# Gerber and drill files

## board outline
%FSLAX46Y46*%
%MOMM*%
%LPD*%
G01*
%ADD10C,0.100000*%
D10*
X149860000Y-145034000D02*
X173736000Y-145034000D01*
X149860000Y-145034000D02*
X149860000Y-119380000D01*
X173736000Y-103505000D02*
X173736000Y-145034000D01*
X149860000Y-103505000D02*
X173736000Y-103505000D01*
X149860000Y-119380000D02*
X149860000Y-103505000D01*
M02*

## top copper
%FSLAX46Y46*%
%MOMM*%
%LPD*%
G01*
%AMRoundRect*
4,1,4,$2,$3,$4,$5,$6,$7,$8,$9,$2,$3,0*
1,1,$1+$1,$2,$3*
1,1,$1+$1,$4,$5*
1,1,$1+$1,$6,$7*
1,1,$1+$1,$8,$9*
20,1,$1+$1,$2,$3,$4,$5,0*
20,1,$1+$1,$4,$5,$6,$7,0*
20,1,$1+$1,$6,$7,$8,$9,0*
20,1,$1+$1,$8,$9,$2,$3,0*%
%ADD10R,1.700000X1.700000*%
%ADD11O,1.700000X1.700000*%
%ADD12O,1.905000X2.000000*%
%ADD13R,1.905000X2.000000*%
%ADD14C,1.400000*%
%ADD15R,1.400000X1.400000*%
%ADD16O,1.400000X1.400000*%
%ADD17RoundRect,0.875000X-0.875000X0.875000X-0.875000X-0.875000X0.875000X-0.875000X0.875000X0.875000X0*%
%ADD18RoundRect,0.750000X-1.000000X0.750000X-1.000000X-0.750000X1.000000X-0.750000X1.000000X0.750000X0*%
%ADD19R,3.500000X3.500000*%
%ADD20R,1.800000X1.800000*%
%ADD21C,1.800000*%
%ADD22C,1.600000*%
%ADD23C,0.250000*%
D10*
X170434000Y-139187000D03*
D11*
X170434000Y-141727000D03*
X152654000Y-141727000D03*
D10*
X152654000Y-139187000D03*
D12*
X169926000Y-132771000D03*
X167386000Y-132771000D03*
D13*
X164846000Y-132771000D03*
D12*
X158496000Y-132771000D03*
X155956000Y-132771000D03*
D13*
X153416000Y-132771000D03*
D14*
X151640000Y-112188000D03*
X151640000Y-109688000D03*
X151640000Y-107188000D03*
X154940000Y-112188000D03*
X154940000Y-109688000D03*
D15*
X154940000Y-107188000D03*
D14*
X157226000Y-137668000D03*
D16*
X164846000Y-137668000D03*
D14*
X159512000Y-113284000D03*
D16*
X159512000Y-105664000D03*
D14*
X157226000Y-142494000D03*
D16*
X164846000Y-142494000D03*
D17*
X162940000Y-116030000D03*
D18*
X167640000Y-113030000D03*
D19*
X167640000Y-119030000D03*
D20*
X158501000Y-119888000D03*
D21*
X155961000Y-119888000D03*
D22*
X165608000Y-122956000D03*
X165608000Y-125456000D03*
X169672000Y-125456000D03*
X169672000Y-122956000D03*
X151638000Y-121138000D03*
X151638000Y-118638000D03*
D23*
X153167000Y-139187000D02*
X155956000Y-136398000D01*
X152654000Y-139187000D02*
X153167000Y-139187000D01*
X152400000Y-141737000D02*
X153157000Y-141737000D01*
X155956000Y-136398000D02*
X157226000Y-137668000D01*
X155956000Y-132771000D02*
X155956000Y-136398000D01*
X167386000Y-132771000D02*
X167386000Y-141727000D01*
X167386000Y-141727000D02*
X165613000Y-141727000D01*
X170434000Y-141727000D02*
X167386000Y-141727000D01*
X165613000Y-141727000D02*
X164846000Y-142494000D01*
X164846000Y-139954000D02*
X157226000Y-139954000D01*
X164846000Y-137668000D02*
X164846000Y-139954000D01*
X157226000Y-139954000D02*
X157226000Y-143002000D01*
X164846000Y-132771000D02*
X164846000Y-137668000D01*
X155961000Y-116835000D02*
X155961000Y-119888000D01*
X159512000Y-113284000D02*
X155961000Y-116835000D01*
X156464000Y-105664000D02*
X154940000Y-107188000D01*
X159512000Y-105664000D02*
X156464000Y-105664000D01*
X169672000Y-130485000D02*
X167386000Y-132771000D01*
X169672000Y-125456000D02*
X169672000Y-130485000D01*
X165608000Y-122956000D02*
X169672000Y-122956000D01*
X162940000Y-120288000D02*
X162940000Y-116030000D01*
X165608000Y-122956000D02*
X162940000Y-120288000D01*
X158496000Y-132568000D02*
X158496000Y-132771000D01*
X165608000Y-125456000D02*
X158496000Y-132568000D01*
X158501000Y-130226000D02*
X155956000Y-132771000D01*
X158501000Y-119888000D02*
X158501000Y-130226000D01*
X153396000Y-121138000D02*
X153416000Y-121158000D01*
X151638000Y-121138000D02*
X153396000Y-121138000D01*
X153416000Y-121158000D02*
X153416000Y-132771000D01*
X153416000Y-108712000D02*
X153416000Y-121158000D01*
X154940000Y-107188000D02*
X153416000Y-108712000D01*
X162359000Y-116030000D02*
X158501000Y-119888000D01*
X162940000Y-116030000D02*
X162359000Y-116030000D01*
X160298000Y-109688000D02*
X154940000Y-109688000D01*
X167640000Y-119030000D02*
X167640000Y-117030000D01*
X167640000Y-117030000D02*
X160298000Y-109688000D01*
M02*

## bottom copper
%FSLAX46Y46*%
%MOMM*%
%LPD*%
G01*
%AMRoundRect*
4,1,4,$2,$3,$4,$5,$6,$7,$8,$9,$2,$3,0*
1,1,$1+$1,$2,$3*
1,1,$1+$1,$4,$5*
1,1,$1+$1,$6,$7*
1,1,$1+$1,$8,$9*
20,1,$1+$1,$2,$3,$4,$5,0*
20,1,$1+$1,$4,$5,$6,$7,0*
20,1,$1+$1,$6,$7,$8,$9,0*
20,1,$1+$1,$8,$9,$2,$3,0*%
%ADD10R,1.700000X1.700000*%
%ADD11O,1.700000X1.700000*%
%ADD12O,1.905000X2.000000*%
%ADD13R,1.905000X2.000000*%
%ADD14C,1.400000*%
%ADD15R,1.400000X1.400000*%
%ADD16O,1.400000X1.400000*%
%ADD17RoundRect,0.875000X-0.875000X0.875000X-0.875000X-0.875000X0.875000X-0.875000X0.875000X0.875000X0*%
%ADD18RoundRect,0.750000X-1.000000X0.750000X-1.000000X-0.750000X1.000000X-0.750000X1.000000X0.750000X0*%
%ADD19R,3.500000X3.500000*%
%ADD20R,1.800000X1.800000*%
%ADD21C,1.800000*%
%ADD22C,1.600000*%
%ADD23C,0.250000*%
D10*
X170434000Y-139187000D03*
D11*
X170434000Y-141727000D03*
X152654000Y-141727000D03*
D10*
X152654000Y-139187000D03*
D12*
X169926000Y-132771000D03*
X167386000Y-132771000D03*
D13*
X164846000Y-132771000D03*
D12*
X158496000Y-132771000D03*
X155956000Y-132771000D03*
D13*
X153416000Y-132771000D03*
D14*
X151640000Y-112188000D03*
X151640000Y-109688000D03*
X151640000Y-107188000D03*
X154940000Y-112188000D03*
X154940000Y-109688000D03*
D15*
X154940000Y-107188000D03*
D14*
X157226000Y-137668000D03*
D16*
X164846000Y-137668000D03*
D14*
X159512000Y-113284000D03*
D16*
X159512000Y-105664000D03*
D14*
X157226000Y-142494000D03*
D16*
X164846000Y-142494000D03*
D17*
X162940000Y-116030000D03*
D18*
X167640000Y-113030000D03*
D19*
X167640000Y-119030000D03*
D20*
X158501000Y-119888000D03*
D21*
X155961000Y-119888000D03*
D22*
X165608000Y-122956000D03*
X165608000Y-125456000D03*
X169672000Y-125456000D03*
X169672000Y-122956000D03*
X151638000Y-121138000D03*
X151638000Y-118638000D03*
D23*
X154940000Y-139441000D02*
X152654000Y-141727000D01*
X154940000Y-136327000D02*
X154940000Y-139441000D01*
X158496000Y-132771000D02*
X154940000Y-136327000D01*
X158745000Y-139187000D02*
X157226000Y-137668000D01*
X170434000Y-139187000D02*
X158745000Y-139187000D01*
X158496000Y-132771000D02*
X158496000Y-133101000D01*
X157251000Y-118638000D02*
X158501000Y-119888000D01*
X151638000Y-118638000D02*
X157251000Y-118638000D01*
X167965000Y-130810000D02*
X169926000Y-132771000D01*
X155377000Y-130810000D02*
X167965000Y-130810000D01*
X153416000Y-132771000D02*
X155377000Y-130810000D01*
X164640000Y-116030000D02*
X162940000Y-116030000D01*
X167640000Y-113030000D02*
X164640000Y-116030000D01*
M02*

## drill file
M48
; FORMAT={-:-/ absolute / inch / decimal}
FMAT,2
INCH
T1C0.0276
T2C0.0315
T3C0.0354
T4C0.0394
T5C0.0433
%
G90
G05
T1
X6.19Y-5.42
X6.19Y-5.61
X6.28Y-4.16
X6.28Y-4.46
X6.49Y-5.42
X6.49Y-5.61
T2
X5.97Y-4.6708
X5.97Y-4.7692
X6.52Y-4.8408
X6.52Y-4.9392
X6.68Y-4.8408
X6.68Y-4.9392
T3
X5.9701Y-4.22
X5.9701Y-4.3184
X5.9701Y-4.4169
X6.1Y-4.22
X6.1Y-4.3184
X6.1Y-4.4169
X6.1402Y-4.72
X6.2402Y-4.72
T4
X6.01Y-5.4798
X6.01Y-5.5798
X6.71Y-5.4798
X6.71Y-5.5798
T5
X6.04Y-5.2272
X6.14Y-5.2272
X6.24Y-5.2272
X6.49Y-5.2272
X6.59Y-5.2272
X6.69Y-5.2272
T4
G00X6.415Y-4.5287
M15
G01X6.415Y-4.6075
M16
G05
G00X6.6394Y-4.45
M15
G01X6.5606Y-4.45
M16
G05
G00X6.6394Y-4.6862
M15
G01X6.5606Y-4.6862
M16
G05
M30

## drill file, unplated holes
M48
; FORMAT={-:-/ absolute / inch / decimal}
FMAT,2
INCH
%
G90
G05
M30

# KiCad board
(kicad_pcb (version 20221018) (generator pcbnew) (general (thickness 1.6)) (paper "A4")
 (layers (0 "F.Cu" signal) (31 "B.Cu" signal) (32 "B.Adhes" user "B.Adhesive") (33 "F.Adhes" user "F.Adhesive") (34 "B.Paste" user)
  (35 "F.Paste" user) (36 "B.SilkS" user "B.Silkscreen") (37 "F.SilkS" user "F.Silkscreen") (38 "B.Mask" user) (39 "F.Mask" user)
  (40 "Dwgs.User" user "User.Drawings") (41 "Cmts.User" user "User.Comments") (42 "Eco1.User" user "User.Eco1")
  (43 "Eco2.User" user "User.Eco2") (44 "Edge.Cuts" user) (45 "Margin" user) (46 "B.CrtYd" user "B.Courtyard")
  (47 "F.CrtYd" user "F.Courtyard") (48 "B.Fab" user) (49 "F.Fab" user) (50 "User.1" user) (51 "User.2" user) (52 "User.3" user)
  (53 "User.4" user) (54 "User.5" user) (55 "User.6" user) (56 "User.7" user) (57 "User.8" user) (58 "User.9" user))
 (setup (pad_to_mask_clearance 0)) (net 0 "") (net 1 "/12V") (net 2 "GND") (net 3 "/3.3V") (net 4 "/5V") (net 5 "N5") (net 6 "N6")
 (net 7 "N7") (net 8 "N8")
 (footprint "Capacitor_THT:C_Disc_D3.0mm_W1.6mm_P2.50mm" (layer "F.Cu") (at 130.175 116.8835 90)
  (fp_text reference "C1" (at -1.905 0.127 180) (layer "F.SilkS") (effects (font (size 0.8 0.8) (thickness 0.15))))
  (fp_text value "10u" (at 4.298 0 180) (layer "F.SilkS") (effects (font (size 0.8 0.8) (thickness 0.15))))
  (pad "1" thru_hole circle (at 0 0 90) (size 1.6 1.6) (drill 0.8) (layers "*.Cu" "*.Mask") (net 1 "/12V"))
  (pad "2" thru_hole circle (at 2.5 0 90) (size 1.6 1.6) (drill 0.8) (layers "*.Cu" "*.Mask") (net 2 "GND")))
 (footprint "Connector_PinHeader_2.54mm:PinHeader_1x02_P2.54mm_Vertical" (layer "F.Cu") (at 148.971 134.9325)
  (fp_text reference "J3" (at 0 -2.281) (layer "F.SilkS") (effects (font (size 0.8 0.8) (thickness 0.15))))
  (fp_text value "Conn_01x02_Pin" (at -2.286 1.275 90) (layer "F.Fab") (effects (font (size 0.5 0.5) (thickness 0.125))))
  (pad "1" thru_hole rect (at 0 0) (size 1.7 1.7) (drill 1) (layers "*.Cu" "*.Mask") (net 2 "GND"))
  (pad "2" thru_hole oval (at 0 2.54) (size 1.7 1.7) (drill 1) (layers "*.Cu" "*.Mask") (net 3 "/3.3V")))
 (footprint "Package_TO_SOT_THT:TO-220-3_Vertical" (layer "F.Cu") (at 131.953 128.5165)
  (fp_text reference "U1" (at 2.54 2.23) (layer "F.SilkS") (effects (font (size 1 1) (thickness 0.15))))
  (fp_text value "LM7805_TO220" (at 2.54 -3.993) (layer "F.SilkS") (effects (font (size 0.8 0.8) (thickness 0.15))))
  (pad "1" thru_hole rect (at 0 0) (size 1.905 2) (drill 1.1) (layers "*.Cu" "*.Mask") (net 1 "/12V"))
  (pad "2" thru_hole oval (at 2.54 0) (size 1.905 2) (drill 1.1) (layers "*.Cu" "*.Mask") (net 2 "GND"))
  (pad "3" thru_hole oval (at 5.08 0) (size 1.905 2) (drill 1.1) (layers "*.Cu" "*.Mask") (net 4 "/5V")))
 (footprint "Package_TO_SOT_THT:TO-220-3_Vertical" (layer "F.Cu") (at 143.383 128.5165)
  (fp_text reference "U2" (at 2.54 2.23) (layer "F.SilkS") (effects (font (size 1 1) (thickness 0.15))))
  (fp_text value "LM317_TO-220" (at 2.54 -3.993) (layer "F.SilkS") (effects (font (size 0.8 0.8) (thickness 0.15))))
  (pad "1" thru_hole rect (at 0 0) (size 1.905 2) (drill 1.1) (layers "*.Cu" "*.Mask") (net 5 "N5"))
  (pad "2" thru_hole oval (at 2.54 0) (size 1.905 2) (drill 1.1) (layers "*.Cu" "*.Mask") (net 3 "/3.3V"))
  (pad "3" thru_hole oval (at 5.08 0) (size 1.905 2) (drill 1.1) (layers "*.Cu" "*.Mask") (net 1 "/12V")))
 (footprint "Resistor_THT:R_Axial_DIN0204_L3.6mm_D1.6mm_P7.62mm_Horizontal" (layer "F.Cu") (at 135.763 138.2395)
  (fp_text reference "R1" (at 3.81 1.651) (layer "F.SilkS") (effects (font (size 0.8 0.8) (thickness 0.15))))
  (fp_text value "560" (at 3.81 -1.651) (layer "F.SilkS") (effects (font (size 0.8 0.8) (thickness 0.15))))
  (pad "1" thru_hole circle (at 0 0) (size 1.4 1.4) (drill 0.7) (layers "*.Cu" "*.Mask") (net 5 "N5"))
  (pad "2" thru_hole oval (at 7.62 0) (size 1.4 1.4) (drill 0.7) (layers "*.Cu" "*.Mask") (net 3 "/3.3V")))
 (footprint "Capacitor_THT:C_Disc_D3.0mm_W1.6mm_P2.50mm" (layer "F.Cu") (at 148.209 121.2015 90)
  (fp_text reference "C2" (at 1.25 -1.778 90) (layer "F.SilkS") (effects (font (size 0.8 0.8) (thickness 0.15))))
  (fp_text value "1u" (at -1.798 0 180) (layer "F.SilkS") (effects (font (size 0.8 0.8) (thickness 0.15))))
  (pad "1" thru_hole circle (at 0 0 90) (size 1.6 1.6) (drill 0.8) (layers "*.Cu" "*.Mask") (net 3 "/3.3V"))
  (pad "2" thru_hole circle (at 2.5 0 90) (size 1.6 1.6) (drill 0.8) (layers "*.Cu" "*.Mask") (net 2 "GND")))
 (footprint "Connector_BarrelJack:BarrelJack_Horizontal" (layer "F.Cu") (at 146.177 114.7755 -90)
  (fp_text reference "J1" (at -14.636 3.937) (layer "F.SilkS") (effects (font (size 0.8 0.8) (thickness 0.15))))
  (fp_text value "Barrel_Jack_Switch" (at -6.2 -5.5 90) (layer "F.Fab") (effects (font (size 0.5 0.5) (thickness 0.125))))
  (pad "1" thru_hole rect (at 0 0 270) (size 3.5 3.5) (drill oval 1 3) (layers "*.Cu" "*.Mask") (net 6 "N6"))
  (pad "2" thru_hole roundrect (at -6 0 270) (size 3 3.5) (drill oval 1 3) (layers "*.Cu" "*.Mask") (roundrect_rratio 0.25) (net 2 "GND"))
  (pad "3" thru_hole roundrect (at -3 4.7 270) (size 3.5 3.5) (drill oval 3 1) (layers "*.Cu" "*.Mask") (roundrect_rratio 0.25)
   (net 2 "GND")))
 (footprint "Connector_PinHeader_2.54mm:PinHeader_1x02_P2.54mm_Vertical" (layer "F.Cu") (at 131.191 134.9325)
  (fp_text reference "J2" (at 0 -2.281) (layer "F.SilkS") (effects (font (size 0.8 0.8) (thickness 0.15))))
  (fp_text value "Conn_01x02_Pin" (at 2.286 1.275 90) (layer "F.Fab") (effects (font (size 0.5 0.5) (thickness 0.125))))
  (pad "1" thru_hole rect (at 0 0) (size 1.7 1.7) (drill 1) (layers "*.Cu" "*.Mask") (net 2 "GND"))
  (pad "2" thru_hole oval (at 0 2.54) (size 1.7 1.7) (drill 1) (layers "*.Cu" "*.Mask") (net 4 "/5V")))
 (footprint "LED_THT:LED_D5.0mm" (layer "F.Cu") (at 137.038 115.6335 180)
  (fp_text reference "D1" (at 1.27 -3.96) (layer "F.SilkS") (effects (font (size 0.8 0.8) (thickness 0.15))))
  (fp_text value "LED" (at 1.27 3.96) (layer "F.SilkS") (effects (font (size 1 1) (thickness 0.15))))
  (pad "1" thru_hole rect (at 0 0 180) (size 1.8 1.8) (drill 0.9) (layers "*.Cu" "*.Mask") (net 2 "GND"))
  (pad "2" thru_hole circle (at 2.54 0 180) (size 1.8 1.8) (drill 0.9) (layers "*.Cu" "*.Mask") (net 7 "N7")))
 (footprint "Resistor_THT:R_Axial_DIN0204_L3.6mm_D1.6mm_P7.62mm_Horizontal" (layer "F.Cu") (at 135.763 133.4135)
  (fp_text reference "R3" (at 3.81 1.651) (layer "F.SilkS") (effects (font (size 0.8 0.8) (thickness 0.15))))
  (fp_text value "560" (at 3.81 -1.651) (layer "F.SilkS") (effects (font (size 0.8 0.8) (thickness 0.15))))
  (pad "1" thru_hole circle (at 0 0) (size 1.4 1.4) (drill 0.7) (layers "*.Cu" "*.Mask") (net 2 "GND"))
  (pad "2" thru_hole oval (at 7.62 0) (size 1.4 1.4) (drill 0.7) (layers "*.Cu" "*.Mask") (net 5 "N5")))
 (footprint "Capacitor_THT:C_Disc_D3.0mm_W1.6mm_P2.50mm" (layer "F.Cu") (at 144.145 121.2015 90)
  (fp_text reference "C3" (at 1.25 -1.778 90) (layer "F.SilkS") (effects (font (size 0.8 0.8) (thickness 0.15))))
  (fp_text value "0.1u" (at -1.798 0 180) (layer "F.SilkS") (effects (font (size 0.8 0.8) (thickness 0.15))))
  (pad "1" thru_hole circle (at 0 0 90) (size 1.6 1.6) (drill 0.8) (layers "*.Cu" "*.Mask") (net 4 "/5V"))
  (pad "2" thru_hole circle (at 2.5 0 90) (size 1.6 1.6) (drill 0.8) (layers "*.Cu" "*.Mask") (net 2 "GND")))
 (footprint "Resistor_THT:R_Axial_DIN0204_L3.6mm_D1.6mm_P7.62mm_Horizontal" (layer "F.Cu") (at 138.049 109.0295 90)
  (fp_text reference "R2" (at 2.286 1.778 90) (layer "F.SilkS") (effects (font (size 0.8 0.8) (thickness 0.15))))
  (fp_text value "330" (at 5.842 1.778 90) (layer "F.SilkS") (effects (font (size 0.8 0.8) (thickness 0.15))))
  (pad "1" thru_hole circle (at 0 0 90) (size 1.4 1.4) (drill 0.7) (layers "*.Cu" "*.Mask") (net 7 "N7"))
  (pad "2" thru_hole oval (at 7.62 0 90) (size 1.4 1.4) (drill 0.7) (layers "*.Cu" "*.Mask") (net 1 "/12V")))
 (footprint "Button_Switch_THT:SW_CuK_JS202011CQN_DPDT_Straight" (layer "F.Cu") (at 133.477 102.9335 -90)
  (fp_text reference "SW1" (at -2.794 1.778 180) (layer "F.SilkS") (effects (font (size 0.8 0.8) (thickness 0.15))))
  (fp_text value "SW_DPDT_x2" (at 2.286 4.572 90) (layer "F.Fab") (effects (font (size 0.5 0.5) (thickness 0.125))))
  (pad "1" thru_hole rect (at 0 0 270) (size 1.4 1.4) (drill 0.9) (layers "*.Cu" "*.Mask") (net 1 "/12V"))
  (pad "2" thru_hole circle (at 2.5 0 270) (size 1.4 1.4) (drill 0.9) (layers "*.Cu" "*.Mask") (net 6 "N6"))
  (pad "3" thru_hole circle (at 5 0 270) (size 1.4 1.4) (drill 0.9) (layers "*.Cu" "*.Mask") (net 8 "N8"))
  (pad "4" thru_hole circle (at 0 3.3 270) (size 1.4 1.4) (drill 0.9) (layers "*.Cu" "*.Mask"))
  (pad "5" thru_hole circle (at 2.5 3.3 270) (size 1.4 1.4) (drill 0.9) (layers "*.Cu" "*.Mask"))
  (pad "6" thru_hole circle (at 5 3.3 270) (size 1.4 1.4) (drill 0.9) (layers "*.Cu" "*.Mask")))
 (gr_line (start 128.397 115.1255) (end 128.397 99.2505) (stroke (width 0.1) (type default)) (layer "Edge.Cuts"))
 (gr_line (start 128.397 140.7795) (end 152.273 140.7795) (stroke (width 0.1) (type default)) (layer "Edge.Cuts"))
 (gr_line (start 152.273 99.2505) (end 152.273 140.7795) (stroke (width 0.1) (type default)) (layer "Edge.Cuts"))
 (gr_line (start 128.397 140.7795) (end 128.397 115.1255) (stroke (width 0.1) (type default)) (layer "Edge.Cuts"))
 (gr_line (start 128.397 99.2505) (end 152.273 99.2505) (stroke (width 0.1) (type default)) (layer "Edge.Cuts"))
 (segment (start 135.001 101.4095) (end 133.477 102.9335) (width 0.25) (layer "F.Cu") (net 1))
 (segment (start 131.933 116.8835) (end 131.953 116.9035) (width 0.25) (layer "F.Cu") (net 1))
 (segment (start 131.953 104.4575) (end 131.953 116.9035) (width 0.25) (layer "F.Cu") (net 1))
 (segment (start 138.049 101.4095) (end 135.001 101.4095) (width 0.25) (layer "F.Cu") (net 1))
 (segment (start 133.477 102.9335) (end 131.953 104.4575) (width 0.25) (layer "F.Cu") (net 1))
 (segment (start 131.953 116.9035) (end 131.953 128.5165) (width 0.25) (layer "F.Cu") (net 1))
 (segment (start 130.175 116.8835) (end 131.933 116.8835) (width 0.25) (layer "F.Cu") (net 1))
 (segment (start 133.914 126.5555) (end 146.502 126.5555) (width 0.25) (layer "B.Cu") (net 1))
 (segment (start 131.953 128.5165) (end 133.914 126.5555) (width 0.25) (layer "B.Cu") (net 1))
 (segment (start 146.502 126.5555) (end 148.463 128.5165) (width 0.25) (layer "B.Cu") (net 1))
 (segment (start 141.477 111.7755) (end 140.896 111.7755) (width 0.25) (layer "F.Cu") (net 2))
 (segment (start 144.145 118.7015) (end 141.477 116.0335) (width 0.25) (layer "F.Cu") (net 2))
 (segment (start 134.493 132.1435) (end 135.763 133.4135) (width 0.25) (layer "F.Cu") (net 2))
 (segment (start 137.038 115.6335) (end 137.038 125.9715) (width 0.25) (layer "F.Cu") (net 2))
 (segment (start 137.038 125.9715) (end 134.493 128.5165) (width 0.25) (layer "F.Cu") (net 2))
 (segment (start 131.191 134.9325) (end 131.704 134.9325) (width 0.25) (layer "F.Cu") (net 2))
 (segment (start 134.493 128.5165) (end 134.493 132.1435) (width 0.25) (layer "F.Cu") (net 2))
 (segment (start 140.896 111.7755) (end 137.038 115.6335) (width 0.25) (layer "F.Cu") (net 2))
 (segment (start 144.145 118.7015) (end 148.209 118.7015) (width 0.25) (layer "F.Cu") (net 2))
 (segment (start 141.477 116.0335) (end 141.477 111.7755) (width 0.25) (layer "F.Cu") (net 2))
 (segment (start 131.704 134.9325) (end 134.493 132.1435) (width 0.25) (layer "F.Cu") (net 2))
 (segment (start 130.175 114.3835) (end 135.788 114.3835) (width 0.25) (layer "B.Cu") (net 2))
 (segment (start 137.282 134.9325) (end 135.763 133.4135) (width 0.25) (layer "B.Cu") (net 2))
 (segment (start 148.971 134.9325) (end 137.282 134.9325) (width 0.25) (layer "B.Cu") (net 2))
 (segment (start 135.788 114.3835) (end 137.038 115.6335) (width 0.25) (layer "B.Cu") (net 2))
 (segment (start 146.177 108.7755) (end 143.177 111.7755) (width 0.25) (layer "B.Cu") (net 2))
 (segment (start 143.177 111.7755) (end 141.477 111.7755) (width 0.25) (layer "B.Cu") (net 2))
 (segment (start 148.971 137.4725) (end 145.923 137.4725) (width 0.25) (layer "F.Cu") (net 3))
 (segment (start 148.209 121.2015) (end 148.209 126.2305) (width 0.25) (layer "F.Cu") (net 3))
 (segment (start 148.209 126.2305) (end 145.923 128.5165) (width 0.25) (layer "F.Cu") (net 3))
 (segment (start 145.923 128.5165) (end 145.923 137.4725) (width 0.25) (layer "F.Cu") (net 3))
 (segment (start 144.15 137.4725) (end 143.383 138.2395) (width 0.25) (layer "F.Cu") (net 3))
 (segment (start 145.923 137.4725) (end 144.15 137.4725) (width 0.25) (layer "F.Cu") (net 3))
 (segment (start 144.145 121.2015) (end 137.033 128.3135) (width 0.25) (layer "F.Cu") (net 4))
 (segment (start 137.033 128.3135) (end 137.033 128.5165) (width 0.25) (layer "F.Cu") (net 4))
 (segment (start 130.937 137.4825) (end 131.694 137.4825) (width 0.25) (layer "F.Cu") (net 4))
 (segment (start 137.033 128.5165) (end 137.033 128.8465) (width 0.25) (layer "B.Cu") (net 4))
 (segment (start 133.477 135.1865) (end 131.191 137.4725) (width 0.25) (layer "B.Cu") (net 4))
 (segment (start 137.033 128.5165) (end 133.477 132.0725) (width 0.25) (layer "B.Cu") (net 4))
 (segment (start 133.477 132.0725) (end 133.477 135.1865) (width 0.25) (layer "B.Cu") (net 4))
 (segment (start 134.498 112.5805) (end 134.498 115.6335) (width 0.25) (layer "F.Cu") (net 7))
 (segment (start 138.049 109.0295) (end 134.498 112.5805) (width 0.25) (layer "F.Cu") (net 7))
 (segment (start 138.835 105.4335) (end 133.477 105.4335) (width 0.25) (layer "F.Cu") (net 6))
 (segment (start 146.177 112.7755) (end 138.835 105.4335) (width 0.25) (layer "F.Cu") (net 6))
 (segment (start 146.177 114.7755) (end 146.177 112.7755) (width 0.25) (layer "F.Cu") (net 6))
 (segment (start 135.763 135.6995) (end 135.763 138.7475) (width 0.25) (layer "F.Cu") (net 5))
 (segment (start 143.383 133.4135) (end 143.383 135.6995) (width 0.25) (layer "F.Cu") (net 5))
 (segment (start 143.383 135.6995) (end 135.763 135.6995) (width 0.25) (layer "F.Cu") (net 5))
 (segment (start 143.383 128.5165) (end 143.383 133.4135) (width 0.25) (layer "F.Cu") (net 5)))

